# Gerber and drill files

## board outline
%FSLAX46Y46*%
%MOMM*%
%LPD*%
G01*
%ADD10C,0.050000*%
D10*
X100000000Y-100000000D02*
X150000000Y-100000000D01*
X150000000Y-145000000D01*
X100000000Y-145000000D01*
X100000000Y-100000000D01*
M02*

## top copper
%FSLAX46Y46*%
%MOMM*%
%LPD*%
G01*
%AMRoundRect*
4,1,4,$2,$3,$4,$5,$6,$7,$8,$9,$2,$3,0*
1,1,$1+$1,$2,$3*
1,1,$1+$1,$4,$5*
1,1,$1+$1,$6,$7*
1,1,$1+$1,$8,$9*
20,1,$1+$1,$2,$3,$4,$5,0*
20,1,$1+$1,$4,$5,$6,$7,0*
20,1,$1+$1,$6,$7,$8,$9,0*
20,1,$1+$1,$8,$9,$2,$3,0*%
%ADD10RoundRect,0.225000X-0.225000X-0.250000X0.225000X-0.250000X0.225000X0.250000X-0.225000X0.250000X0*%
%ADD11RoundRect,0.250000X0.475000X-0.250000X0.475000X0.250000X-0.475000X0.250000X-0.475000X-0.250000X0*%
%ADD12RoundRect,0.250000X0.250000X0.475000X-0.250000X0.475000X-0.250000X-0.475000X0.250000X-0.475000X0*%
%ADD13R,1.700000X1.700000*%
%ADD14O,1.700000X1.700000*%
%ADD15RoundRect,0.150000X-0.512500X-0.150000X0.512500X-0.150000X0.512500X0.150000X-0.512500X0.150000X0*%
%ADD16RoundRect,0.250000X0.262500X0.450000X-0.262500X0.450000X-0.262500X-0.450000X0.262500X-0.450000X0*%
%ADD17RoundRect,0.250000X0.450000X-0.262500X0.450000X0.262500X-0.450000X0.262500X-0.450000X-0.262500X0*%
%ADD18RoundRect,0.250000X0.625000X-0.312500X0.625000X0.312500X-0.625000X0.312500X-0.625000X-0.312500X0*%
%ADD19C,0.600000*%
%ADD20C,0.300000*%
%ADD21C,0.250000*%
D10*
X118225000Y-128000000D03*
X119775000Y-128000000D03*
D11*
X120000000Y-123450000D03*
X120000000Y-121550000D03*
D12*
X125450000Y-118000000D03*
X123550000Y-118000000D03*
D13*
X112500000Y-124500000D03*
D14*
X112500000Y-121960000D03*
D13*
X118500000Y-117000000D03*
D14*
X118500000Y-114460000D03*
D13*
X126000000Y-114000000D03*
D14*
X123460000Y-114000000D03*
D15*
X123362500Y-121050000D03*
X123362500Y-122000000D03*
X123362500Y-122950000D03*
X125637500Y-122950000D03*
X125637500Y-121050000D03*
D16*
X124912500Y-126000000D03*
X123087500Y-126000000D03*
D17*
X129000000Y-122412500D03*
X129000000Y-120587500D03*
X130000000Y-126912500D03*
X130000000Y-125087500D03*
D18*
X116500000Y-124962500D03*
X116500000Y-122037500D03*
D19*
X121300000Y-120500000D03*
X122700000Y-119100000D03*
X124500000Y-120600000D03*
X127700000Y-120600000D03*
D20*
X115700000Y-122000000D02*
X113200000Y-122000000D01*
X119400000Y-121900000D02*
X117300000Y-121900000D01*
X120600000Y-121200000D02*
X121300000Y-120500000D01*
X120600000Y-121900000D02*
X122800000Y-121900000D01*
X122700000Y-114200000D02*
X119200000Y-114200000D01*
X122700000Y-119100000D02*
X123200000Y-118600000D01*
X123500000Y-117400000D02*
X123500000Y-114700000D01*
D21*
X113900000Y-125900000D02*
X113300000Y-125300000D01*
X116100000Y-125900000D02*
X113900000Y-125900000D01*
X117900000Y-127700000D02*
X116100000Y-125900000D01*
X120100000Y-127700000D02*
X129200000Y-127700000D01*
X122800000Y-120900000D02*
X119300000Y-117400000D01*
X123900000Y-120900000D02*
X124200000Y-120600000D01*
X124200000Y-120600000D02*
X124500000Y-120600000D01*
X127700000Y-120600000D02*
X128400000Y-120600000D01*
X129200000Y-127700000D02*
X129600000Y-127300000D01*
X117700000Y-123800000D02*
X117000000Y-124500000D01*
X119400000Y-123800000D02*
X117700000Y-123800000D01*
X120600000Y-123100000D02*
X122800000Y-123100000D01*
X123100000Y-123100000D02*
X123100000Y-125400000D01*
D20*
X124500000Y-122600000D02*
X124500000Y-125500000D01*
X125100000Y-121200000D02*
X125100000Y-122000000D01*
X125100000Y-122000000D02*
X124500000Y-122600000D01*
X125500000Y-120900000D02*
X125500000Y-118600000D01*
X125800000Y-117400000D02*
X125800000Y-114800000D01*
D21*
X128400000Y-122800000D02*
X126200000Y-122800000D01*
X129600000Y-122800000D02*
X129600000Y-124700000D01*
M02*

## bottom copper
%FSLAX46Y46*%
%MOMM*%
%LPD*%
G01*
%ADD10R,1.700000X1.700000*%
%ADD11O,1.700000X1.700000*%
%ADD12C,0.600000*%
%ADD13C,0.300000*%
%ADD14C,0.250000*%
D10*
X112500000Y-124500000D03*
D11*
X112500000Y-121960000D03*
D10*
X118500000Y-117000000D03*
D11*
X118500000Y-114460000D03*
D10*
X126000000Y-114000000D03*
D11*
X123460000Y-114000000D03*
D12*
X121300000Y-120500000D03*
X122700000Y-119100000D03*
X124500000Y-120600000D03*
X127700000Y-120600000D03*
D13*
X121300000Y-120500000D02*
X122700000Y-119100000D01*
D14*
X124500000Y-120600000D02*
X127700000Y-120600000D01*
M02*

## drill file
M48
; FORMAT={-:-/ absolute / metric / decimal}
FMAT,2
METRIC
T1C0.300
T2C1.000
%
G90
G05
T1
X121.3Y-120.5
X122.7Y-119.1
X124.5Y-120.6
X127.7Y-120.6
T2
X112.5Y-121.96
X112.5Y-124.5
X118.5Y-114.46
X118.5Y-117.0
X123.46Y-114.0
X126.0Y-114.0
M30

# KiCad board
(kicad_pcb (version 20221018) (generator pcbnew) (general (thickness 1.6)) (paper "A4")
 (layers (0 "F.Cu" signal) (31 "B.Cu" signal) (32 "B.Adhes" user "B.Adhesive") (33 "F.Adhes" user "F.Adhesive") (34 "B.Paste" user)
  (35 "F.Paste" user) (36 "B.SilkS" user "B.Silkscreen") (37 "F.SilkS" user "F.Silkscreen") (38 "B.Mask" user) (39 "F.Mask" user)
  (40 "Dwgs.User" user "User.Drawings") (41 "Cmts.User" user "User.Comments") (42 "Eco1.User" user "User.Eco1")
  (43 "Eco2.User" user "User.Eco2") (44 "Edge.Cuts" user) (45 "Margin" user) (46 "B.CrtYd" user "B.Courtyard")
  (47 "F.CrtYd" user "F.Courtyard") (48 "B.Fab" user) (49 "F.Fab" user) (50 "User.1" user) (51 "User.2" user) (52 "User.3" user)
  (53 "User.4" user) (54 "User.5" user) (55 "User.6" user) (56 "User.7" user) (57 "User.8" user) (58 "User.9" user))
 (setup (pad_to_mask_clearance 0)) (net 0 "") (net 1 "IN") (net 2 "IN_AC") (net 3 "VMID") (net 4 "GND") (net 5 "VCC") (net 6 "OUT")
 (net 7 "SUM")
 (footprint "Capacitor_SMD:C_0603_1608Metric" (layer "F.Cu") (at 119 128)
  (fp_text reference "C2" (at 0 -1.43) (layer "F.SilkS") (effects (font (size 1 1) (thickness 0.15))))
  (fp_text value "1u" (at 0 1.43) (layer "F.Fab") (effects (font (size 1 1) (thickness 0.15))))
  (pad "1" smd roundrect (at -0.775 0) (size 0.9 0.95) (layers "F.Cu" "F.Paste" "F.Mask") (roundrect_rratio 0.25) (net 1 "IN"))
  (pad "2" smd roundrect (at 0.775 0) (size 0.9 0.95) (layers "F.Cu" "F.Paste" "F.Mask") (roundrect_rratio 0.25) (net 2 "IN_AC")))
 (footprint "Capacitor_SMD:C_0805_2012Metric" (layer "F.Cu") (at 120 122.5 90)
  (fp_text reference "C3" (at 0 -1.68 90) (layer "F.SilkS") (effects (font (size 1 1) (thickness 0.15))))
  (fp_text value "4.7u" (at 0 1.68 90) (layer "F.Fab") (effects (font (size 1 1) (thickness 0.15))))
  (pad "1" smd roundrect (at -0.95 0 90) (size 1 1.45) (layers "F.Cu" "F.Paste" "F.Mask") (roundrect_rratio 0.25) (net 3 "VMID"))
  (pad "2" smd roundrect (at 0.95 0 90) (size 1 1.45) (layers "F.Cu" "F.Paste" "F.Mask") (roundrect_rratio 0.25) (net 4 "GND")))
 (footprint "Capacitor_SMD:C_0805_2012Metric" (layer "F.Cu") (at 124.5 118 180)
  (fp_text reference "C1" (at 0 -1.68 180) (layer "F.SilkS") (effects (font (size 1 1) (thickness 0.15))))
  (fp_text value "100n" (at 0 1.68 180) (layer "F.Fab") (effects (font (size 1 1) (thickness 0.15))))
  (pad "1" smd roundrect (at -0.95 0 180) (size 1 1.45) (layers "F.Cu" "F.Paste" "F.Mask") (roundrect_rratio 0.25) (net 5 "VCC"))
  (pad "2" smd roundrect (at 0.95 0 180) (size 1 1.45) (layers "F.Cu" "F.Paste" "F.Mask") (roundrect_rratio 0.25) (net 4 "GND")))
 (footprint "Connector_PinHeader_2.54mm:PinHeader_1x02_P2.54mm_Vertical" (layer "F.Cu") (at 112.5 124.5 180)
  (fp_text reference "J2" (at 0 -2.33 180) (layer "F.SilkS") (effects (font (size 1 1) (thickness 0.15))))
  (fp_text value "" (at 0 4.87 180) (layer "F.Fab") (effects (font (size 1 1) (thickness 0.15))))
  (pad "1" thru_hole rect (at 0 0 180) (size 1.7 1.7) (drill 1) (layers "*.Cu" "*.Mask") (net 1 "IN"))
  (pad "2" thru_hole oval (at 0 2.54 180) (size 1.7 1.7) (drill 1) (layers "*.Cu" "*.Mask") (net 4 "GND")))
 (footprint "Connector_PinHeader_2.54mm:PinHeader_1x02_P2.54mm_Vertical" (layer "F.Cu") (at 118.5 117 180)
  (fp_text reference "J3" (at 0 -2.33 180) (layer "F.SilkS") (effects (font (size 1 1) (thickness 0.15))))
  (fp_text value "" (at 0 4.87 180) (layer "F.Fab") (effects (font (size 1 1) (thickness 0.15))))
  (pad "1" thru_hole rect (at 0 0 180) (size 1.7 1.7) (drill 1) (layers "*.Cu" "*.Mask") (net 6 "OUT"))
  (pad "2" thru_hole oval (at 0 2.54 180) (size 1.7 1.7) (drill 1) (layers "*.Cu" "*.Mask") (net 4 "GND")))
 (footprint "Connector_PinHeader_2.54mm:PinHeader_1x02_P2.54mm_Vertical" (layer "F.Cu") (at 126 114 -90)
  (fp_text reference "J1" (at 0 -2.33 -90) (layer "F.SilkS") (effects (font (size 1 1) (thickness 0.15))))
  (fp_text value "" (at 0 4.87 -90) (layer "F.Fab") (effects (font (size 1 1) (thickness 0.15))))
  (pad "1" thru_hole rect (at 0 0 270) (size 1.7 1.7) (drill 1) (layers "*.Cu" "*.Mask") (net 5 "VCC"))
  (pad "2" thru_hole oval (at 0 2.54 270) (size 1.7 1.7) (drill 1) (layers "*.Cu" "*.Mask") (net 4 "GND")))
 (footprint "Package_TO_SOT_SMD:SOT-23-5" (layer "F.Cu") (at 124.5 122)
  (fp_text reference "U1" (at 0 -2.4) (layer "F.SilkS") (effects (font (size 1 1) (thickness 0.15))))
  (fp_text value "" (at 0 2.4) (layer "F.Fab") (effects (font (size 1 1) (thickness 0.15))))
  (pad "1" smd roundrect (at -1.1375 -0.95) (size 1.325 0.6) (layers "F.Cu" "F.Paste" "F.Mask") (roundrect_rratio 0.25) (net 6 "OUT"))
  (pad "2" smd roundrect (at -1.1375 0) (size 1.325 0.6) (layers "F.Cu" "F.Paste" "F.Mask") (roundrect_rratio 0.25) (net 4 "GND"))
  (pad "3" smd roundrect (at -1.1375 0.95) (size 1.325 0.6) (layers "F.Cu" "F.Paste" "F.Mask") (roundrect_rratio 0.25) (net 3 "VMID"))
  (pad "4" smd roundrect (at 1.1375 0.95) (size 1.325 0.6) (layers "F.Cu" "F.Paste" "F.Mask") (roundrect_rratio 0.25) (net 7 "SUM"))
  (pad "5" smd roundrect (at 1.1375 -0.95) (size 1.325 0.6) (layers "F.Cu" "F.Paste" "F.Mask") (roundrect_rratio 0.25) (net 5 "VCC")))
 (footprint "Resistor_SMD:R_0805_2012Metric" (layer "F.Cu") (at 124 126 180)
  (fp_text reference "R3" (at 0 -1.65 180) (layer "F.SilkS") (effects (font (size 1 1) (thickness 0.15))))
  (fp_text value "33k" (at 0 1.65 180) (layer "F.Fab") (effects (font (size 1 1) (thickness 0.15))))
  (pad "1" smd roundrect (at -0.9125 0 180) (size 1.025 1.4) (layers "F.Cu" "F.Paste" "F.Mask") (roundrect_rratio 0.243902) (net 5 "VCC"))
  (pad "2" smd roundrect (at 0.9125 0 180) (size 1.025 1.4) (layers "F.Cu" "F.Paste" "F.Mask") (roundrect_rratio 0.243902) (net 3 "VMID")))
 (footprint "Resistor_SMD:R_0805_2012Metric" (layer "F.Cu") (at 129 121.5 90)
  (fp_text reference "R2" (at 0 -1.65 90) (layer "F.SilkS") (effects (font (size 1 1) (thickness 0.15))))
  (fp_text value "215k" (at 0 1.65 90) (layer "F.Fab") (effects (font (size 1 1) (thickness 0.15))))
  (pad "1" smd roundrect (at -0.9125 0 90) (size 1.025 1.4) (layers "F.Cu" "F.Paste" "F.Mask") (roundrect_rratio 0.243902) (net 7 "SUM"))
  (pad "2" smd roundrect (at 0.9125 0 90) (size 1.025 1.4) (layers "F.Cu" "F.Paste" "F.Mask") (roundrect_rratio 0.243902) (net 6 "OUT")))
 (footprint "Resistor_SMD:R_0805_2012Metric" (layer "F.Cu") (at 130 126 90)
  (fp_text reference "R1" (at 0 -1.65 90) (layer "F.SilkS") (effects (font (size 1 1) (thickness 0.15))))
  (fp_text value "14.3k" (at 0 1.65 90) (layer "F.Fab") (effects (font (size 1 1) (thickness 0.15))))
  (pad "1" smd roundrect (at -0.9125 0 90) (size 1.025 1.4) (layers "F.Cu" "F.Paste" "F.Mask") (roundrect_rratio 0.243902) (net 2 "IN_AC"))
  (pad "2" smd roundrect (at 0.9125 0 90) (size 1.025 1.4) (layers "F.Cu" "F.Paste" "F.Mask") (roundrect_rratio 0.243902) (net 7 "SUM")))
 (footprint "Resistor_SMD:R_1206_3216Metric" (layer "F.Cu") (at 116.5 123.5 90)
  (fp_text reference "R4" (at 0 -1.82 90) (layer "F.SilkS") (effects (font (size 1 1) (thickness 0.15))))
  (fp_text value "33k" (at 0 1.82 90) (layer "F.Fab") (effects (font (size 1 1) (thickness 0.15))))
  (pad "1" smd roundrect (at -1.4625 0 90) (size 1.125 1.75) (layers "F.Cu" "F.Paste" "F.Mask") (roundrect_rratio 0.222222) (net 3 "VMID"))
  (pad "2" smd roundrect (at 1.4625 0 90) (size 1.125 1.75) (layers "F.Cu" "F.Paste" "F.Mask") (roundrect_rratio 0.222222) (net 4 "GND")))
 (gr_rect (start 100 100) (end 150 145) (stroke (width 0.05) (type default)) (fill none) (layer "Edge.Cuts"))
 (segment (start 115.7 122) (end 113.2 122) (width 0.3) (layer "F.Cu") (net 4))
 (segment (start 119.4 121.9) (end 117.3 121.9) (width 0.3) (layer "F.Cu") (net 4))
 (segment (start 120.6 121.2) (end 121.3 120.5) (width 0.3) (layer "F.Cu") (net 4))
 (segment (start 120.6 121.9) (end 122.8 121.9) (width 0.3) (layer "F.Cu") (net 4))
 (segment (start 122.7 114.2) (end 119.2 114.2) (width 0.3) (layer "F.Cu") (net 4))
 (segment (start 122.7 119.1) (end 123.2 118.6) (width 0.3) (layer "F.Cu") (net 4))
 (segment (start 123.5 117.4) (end 123.5 114.7) (width 0.3) (layer "F.Cu") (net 4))
 (via (at 121.3 120.5) (size 0.6) (drill 0.3) (layers "F.Cu" "B.Cu") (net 4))
 (via (at 122.7 119.1) (size 0.6) (drill 0.3) (layers "F.Cu" "B.Cu") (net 4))
 (segment (start 113.9 125.9) (end 113.3 125.3) (width 0.25) (layer "F.Cu") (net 1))
 (segment (start 116.1 125.9) (end 113.9 125.9) (width 0.25) (layer "F.Cu") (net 1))
 (segment (start 117.9 127.7) (end 116.1 125.9) (width 0.25) (layer "F.Cu") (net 1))
 (segment (start 120.1 127.7) (end 129.2 127.7) (width 0.25) (layer "F.Cu") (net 2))
 (segment (start 121.3 120.5) (end 122.7 119.1) (width 0.3) (layer "B.Cu") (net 4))
 (segment (start 122.8 120.9) (end 119.3 117.4) (width 0.25) (layer "F.Cu") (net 6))
 (segment (start 123.9 120.9) (end 124.2 120.6) (width 0.25) (layer "F.Cu") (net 6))
 (segment (start 124.2 120.6) (end 124.5 120.6) (width 0.25) (layer "F.Cu") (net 6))
 (segment (start 127.7 120.6) (end 128.4 120.6) (width 0.25) (layer "F.Cu") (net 6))
 (segment (start 129.2 127.7) (end 129.6 127.3) (width 0.25) (layer "F.Cu") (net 2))
 (via (at 124.5 120.6) (size 0.6) (drill 0.3) (layers "F.Cu" "B.Cu") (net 6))
 (via (at 127.7 120.6) (size 0.6) (drill 0.3) (layers "F.Cu" "B.Cu") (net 6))
 (segment (start 117.7 123.8) (end 117 124.5) (width 0.25) (layer "F.Cu") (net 3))
 (segment (start 119.4 123.8) (end 117.7 123.8) (width 0.25) (layer "F.Cu") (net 3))
 (segment (start 120.6 123.1) (end 122.8 123.1) (width 0.25) (layer "F.Cu") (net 3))
 (segment (start 123.1 123.1) (end 123.1 125.4) (width 0.25) (layer "F.Cu") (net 3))
 (segment (start 124.5 120.6) (end 127.7 120.6) (width 0.25) (layer "B.Cu") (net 6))
 (segment (start 124.5 122.6) (end 124.5 125.5) (width 0.3) (layer "F.Cu") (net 5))
 (segment (start 125.1 121.2) (end 125.1 122) (width 0.3) (layer "F.Cu") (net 5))
 (segment (start 125.1 122) (end 124.5 122.6) (width 0.3) (layer "F.Cu") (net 5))
 (segment (start 125.5 120.9) (end 125.5 118.6) (width 0.3) (layer "F.Cu") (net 5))
 (segment (start 125.8 117.4) (end 125.8 114.8) (width 0.3) (layer "F.Cu") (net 5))
 (segment (start 128.4 122.8) (end 126.2 122.8) (width 0.25) (layer "F.Cu") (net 7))
 (segment (start 129.6 122.8) (end 129.6 124.7) (width 0.25) (layer "F.Cu") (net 7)))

